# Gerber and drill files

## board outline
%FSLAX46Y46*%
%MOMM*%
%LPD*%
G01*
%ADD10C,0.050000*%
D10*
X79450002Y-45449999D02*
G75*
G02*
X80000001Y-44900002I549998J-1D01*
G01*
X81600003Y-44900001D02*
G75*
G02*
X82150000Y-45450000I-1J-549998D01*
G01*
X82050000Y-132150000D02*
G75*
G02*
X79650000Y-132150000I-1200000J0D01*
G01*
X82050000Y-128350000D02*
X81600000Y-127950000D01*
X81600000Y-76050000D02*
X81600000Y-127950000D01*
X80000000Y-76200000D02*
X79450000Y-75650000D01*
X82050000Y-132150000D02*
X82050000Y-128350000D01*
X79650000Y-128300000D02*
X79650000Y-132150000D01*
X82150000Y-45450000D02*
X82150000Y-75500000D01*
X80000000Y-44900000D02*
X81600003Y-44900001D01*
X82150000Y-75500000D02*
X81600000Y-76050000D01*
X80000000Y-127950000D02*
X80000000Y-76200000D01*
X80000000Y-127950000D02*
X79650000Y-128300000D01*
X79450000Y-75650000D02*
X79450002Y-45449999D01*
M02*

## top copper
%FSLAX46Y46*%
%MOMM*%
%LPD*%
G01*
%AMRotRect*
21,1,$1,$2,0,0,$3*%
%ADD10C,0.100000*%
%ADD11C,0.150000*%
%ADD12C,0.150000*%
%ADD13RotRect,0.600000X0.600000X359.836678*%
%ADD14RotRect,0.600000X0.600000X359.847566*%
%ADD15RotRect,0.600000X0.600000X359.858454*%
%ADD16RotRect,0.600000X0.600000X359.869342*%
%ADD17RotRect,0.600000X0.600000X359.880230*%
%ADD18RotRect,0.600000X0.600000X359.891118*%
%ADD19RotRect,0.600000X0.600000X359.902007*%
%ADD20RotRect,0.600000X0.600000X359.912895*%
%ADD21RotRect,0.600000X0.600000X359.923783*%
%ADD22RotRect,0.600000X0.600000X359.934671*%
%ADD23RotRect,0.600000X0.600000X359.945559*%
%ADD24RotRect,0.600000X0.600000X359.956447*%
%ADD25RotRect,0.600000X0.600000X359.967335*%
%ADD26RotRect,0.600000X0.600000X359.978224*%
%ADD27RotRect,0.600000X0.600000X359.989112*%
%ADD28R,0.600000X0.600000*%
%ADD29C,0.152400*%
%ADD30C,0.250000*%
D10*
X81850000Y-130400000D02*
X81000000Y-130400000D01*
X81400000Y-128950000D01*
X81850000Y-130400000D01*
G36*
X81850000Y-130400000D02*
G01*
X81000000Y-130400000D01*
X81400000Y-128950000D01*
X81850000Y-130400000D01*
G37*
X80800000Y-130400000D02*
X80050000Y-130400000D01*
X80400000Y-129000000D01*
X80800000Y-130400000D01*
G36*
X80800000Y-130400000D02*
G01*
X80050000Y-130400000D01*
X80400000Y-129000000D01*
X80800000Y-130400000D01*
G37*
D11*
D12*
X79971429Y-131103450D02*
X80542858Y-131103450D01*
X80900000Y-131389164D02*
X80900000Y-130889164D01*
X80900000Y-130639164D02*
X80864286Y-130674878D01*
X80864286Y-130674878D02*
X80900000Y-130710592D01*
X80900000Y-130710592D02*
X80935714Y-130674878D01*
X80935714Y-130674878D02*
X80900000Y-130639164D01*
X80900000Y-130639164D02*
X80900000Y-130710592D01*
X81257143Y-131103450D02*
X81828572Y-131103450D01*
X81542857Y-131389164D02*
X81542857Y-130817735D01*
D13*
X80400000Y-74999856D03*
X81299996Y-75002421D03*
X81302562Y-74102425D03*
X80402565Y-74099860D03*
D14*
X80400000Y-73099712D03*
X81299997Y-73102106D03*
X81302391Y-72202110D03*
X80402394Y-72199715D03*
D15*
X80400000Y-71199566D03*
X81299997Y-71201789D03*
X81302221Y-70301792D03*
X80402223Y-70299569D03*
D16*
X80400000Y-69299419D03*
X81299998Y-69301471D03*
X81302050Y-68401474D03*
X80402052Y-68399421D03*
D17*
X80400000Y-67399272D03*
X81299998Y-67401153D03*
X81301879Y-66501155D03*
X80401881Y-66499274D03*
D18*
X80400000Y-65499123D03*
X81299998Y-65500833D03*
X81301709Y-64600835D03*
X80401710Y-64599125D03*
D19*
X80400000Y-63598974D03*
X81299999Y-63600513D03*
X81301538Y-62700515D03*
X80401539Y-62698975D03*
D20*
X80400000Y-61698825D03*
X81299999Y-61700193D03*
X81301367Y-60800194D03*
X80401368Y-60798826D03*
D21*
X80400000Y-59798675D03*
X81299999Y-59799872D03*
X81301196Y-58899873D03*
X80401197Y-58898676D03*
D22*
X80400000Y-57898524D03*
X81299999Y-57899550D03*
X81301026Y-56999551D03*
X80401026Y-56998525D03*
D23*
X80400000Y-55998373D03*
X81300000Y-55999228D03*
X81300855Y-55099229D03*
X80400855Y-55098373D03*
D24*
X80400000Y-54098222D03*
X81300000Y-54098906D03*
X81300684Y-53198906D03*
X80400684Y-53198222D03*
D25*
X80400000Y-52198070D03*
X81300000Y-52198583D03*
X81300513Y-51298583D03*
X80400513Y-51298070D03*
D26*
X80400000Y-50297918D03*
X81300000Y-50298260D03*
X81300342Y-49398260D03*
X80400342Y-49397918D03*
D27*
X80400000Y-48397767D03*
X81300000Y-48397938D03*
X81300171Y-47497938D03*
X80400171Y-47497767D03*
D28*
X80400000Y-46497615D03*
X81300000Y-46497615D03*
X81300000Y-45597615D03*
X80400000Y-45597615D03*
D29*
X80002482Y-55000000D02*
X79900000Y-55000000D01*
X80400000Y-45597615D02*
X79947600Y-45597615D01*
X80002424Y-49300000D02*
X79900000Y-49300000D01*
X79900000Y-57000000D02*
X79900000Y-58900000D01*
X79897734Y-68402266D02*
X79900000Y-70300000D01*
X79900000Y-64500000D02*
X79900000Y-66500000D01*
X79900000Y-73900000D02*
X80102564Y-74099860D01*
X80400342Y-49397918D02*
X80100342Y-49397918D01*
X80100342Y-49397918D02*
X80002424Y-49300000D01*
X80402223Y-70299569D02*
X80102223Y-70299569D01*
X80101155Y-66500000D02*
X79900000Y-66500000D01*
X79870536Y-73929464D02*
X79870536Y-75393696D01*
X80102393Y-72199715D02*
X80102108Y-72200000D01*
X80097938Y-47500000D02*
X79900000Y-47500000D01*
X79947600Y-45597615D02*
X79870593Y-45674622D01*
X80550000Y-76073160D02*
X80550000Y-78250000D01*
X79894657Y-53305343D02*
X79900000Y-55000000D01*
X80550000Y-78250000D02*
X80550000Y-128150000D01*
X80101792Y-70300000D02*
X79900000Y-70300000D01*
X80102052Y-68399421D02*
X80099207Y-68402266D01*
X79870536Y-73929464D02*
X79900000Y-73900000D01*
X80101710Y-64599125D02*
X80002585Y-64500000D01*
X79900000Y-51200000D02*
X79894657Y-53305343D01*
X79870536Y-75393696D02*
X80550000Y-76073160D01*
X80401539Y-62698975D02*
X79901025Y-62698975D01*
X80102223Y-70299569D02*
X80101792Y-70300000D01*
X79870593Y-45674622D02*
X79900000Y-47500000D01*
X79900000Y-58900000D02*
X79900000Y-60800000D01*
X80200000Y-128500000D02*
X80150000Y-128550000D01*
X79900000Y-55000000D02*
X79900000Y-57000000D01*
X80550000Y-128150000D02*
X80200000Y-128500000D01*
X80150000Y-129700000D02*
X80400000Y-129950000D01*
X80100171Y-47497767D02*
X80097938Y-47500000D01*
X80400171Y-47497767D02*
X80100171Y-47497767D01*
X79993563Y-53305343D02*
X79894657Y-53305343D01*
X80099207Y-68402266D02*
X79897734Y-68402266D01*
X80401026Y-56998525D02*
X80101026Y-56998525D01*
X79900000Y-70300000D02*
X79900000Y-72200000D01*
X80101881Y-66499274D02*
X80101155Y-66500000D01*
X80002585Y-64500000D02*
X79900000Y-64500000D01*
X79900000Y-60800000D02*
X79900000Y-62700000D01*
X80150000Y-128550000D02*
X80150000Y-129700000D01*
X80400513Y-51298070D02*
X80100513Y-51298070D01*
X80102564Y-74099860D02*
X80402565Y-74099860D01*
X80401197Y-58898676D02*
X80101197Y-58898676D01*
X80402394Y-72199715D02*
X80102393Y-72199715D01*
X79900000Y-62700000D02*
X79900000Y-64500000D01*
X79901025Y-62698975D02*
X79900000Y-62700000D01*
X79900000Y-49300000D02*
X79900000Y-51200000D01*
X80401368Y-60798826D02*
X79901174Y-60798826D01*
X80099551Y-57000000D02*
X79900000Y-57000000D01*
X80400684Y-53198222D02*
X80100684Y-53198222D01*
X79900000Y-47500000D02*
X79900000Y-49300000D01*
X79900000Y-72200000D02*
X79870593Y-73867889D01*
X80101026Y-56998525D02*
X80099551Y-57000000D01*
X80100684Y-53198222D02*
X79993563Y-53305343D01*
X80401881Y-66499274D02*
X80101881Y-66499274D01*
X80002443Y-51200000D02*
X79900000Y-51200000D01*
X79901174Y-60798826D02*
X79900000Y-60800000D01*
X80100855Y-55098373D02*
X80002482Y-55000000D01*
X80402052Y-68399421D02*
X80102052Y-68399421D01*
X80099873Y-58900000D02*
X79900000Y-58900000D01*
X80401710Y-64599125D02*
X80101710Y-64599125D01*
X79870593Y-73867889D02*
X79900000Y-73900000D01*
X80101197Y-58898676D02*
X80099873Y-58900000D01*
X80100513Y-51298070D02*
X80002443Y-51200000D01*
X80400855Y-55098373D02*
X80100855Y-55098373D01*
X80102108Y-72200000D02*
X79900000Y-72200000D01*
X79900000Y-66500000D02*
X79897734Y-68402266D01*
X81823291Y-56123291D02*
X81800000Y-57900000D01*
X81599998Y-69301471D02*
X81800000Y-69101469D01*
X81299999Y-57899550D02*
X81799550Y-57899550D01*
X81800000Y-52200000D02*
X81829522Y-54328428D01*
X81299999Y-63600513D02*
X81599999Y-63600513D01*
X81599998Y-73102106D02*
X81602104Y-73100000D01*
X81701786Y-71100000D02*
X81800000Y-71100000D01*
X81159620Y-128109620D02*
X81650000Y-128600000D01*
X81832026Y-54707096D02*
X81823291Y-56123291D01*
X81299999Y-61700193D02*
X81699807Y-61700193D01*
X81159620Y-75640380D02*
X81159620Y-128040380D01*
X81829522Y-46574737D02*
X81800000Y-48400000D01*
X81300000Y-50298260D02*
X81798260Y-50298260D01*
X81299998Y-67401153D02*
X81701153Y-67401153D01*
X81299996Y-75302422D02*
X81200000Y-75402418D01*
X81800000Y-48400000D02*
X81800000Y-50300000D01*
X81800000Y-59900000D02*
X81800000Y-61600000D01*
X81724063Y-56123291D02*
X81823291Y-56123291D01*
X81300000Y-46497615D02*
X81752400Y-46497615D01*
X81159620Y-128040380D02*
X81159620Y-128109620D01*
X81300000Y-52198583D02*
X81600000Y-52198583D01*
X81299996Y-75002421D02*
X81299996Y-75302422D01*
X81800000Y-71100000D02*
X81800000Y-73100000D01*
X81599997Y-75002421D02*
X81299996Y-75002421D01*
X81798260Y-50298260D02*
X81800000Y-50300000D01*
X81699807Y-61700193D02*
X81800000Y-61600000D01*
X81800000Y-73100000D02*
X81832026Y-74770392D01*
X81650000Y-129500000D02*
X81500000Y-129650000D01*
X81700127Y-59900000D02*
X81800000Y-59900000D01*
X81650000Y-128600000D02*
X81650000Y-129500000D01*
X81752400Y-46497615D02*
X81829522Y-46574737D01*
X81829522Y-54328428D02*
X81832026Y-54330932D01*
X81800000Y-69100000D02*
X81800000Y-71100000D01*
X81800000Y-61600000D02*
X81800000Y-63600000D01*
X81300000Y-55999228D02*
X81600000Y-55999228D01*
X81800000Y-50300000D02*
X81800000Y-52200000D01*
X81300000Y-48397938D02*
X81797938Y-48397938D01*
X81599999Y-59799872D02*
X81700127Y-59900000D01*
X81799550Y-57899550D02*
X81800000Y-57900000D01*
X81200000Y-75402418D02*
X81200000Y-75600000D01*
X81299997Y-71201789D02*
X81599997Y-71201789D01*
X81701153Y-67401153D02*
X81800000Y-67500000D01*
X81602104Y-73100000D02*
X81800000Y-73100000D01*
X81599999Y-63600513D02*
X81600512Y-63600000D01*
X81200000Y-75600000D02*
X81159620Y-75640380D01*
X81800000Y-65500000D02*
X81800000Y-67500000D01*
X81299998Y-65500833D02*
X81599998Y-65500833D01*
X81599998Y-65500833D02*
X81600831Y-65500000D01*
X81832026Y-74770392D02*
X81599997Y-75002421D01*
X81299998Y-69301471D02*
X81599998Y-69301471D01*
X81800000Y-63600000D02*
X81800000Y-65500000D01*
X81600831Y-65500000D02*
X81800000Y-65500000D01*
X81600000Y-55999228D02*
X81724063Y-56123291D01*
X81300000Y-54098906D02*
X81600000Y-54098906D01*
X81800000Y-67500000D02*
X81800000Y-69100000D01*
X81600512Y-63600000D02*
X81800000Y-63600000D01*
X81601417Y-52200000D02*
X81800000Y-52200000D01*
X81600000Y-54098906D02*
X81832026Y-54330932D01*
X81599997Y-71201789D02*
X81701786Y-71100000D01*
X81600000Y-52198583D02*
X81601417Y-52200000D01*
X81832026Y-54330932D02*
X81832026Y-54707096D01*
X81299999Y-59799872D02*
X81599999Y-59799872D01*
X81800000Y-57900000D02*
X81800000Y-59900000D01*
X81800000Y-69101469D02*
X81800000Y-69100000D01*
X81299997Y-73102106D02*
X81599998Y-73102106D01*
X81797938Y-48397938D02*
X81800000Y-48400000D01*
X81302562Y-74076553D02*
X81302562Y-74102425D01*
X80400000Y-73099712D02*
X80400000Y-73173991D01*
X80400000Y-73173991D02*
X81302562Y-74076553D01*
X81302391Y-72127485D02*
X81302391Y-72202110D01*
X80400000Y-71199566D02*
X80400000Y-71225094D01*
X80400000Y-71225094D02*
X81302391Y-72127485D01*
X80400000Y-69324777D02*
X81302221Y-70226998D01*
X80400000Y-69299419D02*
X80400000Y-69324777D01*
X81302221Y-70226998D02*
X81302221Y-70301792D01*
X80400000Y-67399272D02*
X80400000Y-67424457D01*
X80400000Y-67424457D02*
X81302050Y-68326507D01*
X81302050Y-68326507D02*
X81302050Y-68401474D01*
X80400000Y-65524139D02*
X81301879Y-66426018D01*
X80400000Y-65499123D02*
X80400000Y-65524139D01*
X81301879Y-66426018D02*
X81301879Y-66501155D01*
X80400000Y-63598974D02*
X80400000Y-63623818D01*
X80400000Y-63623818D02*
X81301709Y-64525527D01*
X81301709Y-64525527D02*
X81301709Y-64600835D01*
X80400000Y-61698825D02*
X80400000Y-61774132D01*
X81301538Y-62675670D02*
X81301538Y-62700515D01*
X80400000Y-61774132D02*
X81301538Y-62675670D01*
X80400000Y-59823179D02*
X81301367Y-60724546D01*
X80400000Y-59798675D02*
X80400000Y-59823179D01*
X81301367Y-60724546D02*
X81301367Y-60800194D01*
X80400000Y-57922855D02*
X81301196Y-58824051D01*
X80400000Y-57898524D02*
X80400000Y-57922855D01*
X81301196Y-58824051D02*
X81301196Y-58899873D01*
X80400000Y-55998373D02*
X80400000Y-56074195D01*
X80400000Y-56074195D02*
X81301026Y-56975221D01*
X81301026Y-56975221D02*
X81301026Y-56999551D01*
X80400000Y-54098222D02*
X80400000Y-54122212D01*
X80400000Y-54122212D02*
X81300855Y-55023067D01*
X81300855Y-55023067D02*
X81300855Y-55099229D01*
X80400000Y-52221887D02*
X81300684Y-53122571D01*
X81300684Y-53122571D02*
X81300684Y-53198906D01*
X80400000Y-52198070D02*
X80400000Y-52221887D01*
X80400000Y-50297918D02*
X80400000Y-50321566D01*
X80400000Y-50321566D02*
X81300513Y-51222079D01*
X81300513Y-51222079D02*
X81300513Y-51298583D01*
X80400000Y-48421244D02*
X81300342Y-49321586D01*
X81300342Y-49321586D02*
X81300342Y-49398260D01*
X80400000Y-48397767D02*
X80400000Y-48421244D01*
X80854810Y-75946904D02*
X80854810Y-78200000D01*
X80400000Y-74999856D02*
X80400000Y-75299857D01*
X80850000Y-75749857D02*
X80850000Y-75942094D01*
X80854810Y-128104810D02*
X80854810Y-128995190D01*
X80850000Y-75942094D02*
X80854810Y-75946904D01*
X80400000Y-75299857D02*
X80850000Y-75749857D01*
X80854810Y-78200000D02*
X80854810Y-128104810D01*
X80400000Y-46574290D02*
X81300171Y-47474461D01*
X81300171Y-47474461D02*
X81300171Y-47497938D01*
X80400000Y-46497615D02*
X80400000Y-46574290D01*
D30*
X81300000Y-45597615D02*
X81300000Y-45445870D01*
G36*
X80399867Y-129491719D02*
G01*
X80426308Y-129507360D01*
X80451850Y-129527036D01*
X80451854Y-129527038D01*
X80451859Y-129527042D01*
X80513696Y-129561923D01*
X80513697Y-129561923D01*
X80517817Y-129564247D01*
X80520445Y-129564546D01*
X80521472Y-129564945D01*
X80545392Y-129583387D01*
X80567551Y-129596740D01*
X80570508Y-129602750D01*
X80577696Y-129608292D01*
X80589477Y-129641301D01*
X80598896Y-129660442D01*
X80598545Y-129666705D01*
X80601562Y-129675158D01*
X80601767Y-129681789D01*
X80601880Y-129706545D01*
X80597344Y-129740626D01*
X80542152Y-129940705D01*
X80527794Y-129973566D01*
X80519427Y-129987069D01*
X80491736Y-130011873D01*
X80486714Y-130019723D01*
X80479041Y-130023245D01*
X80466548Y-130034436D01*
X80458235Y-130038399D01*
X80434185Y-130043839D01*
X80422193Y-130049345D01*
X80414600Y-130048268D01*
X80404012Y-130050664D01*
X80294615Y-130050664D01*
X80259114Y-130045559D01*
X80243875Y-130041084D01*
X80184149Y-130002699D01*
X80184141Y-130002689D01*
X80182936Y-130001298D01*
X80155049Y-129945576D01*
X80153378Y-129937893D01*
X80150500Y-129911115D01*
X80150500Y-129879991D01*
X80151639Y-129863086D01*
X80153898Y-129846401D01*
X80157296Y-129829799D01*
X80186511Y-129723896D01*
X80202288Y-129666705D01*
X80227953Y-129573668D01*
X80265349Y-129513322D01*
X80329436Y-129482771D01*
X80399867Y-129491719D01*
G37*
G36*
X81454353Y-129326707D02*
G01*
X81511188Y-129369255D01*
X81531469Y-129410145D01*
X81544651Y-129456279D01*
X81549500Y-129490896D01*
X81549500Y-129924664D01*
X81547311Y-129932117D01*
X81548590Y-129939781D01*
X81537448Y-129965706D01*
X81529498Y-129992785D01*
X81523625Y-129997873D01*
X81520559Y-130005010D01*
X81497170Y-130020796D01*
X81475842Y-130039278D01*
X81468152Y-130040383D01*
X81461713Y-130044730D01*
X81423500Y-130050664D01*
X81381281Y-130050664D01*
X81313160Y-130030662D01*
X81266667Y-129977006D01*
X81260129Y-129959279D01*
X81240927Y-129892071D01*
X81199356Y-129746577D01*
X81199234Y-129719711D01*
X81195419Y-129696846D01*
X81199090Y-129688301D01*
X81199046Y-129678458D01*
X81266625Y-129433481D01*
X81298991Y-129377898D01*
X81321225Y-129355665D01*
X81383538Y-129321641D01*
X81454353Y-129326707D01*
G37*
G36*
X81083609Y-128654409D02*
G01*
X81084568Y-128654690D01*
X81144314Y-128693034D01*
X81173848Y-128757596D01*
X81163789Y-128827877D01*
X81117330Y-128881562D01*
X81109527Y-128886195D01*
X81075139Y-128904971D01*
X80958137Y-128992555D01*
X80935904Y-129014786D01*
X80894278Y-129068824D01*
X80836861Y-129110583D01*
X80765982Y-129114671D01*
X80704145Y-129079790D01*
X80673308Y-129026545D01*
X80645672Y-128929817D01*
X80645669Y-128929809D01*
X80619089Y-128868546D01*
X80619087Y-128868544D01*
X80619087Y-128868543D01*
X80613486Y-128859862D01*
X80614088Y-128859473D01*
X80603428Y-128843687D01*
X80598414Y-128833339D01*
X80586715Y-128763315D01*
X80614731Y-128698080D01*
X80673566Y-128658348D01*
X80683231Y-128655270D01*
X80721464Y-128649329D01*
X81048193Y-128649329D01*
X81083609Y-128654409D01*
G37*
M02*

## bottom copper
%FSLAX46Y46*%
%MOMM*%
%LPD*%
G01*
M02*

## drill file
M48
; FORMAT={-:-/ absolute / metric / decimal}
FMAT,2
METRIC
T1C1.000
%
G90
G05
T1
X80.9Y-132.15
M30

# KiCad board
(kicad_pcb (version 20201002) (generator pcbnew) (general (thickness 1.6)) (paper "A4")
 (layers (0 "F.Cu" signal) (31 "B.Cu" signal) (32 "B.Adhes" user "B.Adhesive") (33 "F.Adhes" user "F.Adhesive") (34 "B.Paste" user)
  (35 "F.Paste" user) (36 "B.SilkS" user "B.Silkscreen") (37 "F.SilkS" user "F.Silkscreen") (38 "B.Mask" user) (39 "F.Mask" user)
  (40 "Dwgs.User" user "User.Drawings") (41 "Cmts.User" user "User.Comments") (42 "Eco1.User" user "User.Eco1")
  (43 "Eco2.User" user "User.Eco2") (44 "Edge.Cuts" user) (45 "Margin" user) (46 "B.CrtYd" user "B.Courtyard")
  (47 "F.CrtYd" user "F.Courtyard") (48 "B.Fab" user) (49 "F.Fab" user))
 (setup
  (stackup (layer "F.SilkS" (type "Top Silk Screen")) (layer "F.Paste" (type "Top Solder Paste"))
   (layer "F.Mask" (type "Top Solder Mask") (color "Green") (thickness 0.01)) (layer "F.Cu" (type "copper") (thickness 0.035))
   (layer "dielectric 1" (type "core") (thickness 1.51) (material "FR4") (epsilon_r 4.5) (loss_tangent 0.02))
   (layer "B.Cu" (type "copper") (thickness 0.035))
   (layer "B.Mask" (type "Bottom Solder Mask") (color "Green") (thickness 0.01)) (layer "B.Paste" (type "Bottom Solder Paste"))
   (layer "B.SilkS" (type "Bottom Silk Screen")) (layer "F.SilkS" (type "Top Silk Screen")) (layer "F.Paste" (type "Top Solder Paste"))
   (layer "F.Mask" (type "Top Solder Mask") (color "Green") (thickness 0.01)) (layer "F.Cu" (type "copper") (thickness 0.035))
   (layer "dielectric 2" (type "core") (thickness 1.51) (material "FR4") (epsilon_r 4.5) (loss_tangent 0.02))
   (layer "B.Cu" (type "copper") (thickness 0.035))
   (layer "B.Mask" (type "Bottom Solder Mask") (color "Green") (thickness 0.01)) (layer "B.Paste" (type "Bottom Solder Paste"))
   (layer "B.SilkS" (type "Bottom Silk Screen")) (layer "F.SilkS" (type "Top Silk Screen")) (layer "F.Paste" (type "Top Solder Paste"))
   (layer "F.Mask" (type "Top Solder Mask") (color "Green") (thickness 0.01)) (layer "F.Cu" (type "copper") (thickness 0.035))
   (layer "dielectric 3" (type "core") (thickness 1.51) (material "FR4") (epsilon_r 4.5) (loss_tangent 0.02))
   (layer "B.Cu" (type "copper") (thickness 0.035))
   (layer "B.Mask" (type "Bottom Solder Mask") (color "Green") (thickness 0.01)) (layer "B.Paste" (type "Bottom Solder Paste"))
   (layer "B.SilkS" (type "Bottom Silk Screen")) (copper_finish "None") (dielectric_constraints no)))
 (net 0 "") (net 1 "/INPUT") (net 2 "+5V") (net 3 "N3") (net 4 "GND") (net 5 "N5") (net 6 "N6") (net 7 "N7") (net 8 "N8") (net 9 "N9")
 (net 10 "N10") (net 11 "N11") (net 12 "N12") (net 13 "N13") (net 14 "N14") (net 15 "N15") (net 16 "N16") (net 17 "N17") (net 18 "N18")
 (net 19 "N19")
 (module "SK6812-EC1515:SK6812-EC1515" (layer "F.Cu") (at 80.4 74.999856 -0.1633223699)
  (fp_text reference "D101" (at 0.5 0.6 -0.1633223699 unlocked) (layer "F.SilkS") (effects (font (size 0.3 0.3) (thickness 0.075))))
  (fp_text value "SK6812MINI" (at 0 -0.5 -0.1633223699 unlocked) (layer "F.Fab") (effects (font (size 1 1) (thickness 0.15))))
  (pad "1" smd rect (at 0 0 359.8366776) (size 0.6 0.6) (layers "F.Cu" "F.Paste" "F.Mask") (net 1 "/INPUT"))
  (pad "2" smd rect (at 0.9 0 359.8366776) (size 0.6 0.6) (layers "F.Cu" "F.Paste" "F.Mask") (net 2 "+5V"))
  (pad "3" smd rect (at 0.9 -0.9 359.8366776) (size 0.6 0.6) (layers "F.Cu" "F.Paste" "F.Mask") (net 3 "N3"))
  (pad "4" smd rect (at 0 -0.9 359.8366776) (size 0.6 0.6) (layers "F.Cu" "F.Paste" "F.Mask") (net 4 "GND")))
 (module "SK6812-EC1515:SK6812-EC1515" (layer "F.Cu") (at 80.4 73.099712 -0.1524342119)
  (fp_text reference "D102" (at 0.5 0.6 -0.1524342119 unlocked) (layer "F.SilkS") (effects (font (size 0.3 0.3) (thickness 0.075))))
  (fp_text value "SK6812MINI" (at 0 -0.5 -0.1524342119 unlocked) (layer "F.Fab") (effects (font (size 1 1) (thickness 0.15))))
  (pad "1" smd rect (at 0 0 359.8475658) (size 0.6 0.6) (layers "F.Cu" "F.Paste" "F.Mask") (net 3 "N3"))
  (pad "2" smd rect (at 0.9 0 359.8475658) (size 0.6 0.6) (layers "F.Cu" "F.Paste" "F.Mask") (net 2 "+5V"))
  (pad "3" smd rect (at 0.9 -0.9 359.8475658) (size 0.6 0.6) (layers "F.Cu" "F.Paste" "F.Mask") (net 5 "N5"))
  (pad "4" smd rect (at 0 -0.9 359.8475658) (size 0.6 0.6) (layers "F.Cu" "F.Paste" "F.Mask") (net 4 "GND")))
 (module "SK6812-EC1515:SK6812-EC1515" (layer "F.Cu") (at 80.4 71.199566 -0.1415460539)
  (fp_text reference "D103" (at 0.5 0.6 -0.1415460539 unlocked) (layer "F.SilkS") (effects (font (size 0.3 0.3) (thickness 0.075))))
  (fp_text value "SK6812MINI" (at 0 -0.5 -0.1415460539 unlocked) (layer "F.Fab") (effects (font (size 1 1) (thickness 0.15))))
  (pad "1" smd rect (at 0 0 359.8584539) (size 0.6 0.6) (layers "F.Cu" "F.Paste" "F.Mask") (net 5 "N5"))
  (pad "2" smd rect (at 0.9 0 359.8584539) (size 0.6 0.6) (layers "F.Cu" "F.Paste" "F.Mask") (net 2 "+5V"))
  (pad "3" smd rect (at 0.9 -0.9 359.8584539) (size 0.6 0.6) (layers "F.Cu" "F.Paste" "F.Mask") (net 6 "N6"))
  (pad "4" smd rect (at 0 -0.9 359.8584539) (size 0.6 0.6) (layers "F.Cu" "F.Paste" "F.Mask") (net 4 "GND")))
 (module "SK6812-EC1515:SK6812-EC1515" (layer "F.Cu") (at 80.4 69.299419 -0.1306578959)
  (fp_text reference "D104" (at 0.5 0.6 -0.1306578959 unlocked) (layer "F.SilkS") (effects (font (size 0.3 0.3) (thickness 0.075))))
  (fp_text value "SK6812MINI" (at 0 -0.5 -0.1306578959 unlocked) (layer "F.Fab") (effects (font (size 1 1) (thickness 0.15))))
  (pad "1" smd rect (at 0 0 359.8693421) (size 0.6 0.6) (layers "F.Cu" "F.Paste" "F.Mask") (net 6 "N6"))
  (pad "2" smd rect (at 0.9 0 359.8693421) (size 0.6 0.6) (layers "F.Cu" "F.Paste" "F.Mask") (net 2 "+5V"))
  (pad "3" smd rect (at 0.9 -0.9 359.8693421) (size 0.6 0.6) (layers "F.Cu" "F.Paste" "F.Mask") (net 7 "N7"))
  (pad "4" smd rect (at 0 -0.9 359.8693421) (size 0.6 0.6) (layers "F.Cu" "F.Paste" "F.Mask") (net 4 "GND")))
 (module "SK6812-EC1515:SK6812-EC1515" (layer "F.Cu") (at 80.4 67.399272 -0.1197697379)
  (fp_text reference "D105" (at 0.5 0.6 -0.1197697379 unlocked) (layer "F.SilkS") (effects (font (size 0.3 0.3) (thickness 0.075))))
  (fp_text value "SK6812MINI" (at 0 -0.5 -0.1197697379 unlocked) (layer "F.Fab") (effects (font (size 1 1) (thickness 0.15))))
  (pad "1" smd rect (at 0 0 359.8802303) (size 0.6 0.6) (layers "F.Cu" "F.Paste" "F.Mask") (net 7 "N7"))
  (pad "2" smd rect (at 0.9 0 359.8802303) (size 0.6 0.6) (layers "F.Cu" "F.Paste" "F.Mask") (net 2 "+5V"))
  (pad "3" smd rect (at 0.9 -0.9 359.8802303) (size 0.6 0.6) (layers "F.Cu" "F.Paste" "F.Mask") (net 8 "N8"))
  (pad "4" smd rect (at 0 -0.9 359.8802303) (size 0.6 0.6) (layers "F.Cu" "F.Paste" "F.Mask") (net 4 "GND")))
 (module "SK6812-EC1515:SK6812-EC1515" (layer "F.Cu") (at 80.4 65.499123 -0.1088815799)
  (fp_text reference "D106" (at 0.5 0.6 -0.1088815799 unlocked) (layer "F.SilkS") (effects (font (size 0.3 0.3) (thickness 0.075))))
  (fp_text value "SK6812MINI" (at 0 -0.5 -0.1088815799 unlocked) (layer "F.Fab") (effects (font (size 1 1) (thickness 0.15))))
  (pad "1" smd rect (at 0 0 359.8911184) (size 0.6 0.6) (layers "F.Cu" "F.Paste" "F.Mask") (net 8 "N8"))
  (pad "2" smd rect (at 0.9 0 359.8911184) (size 0.6 0.6) (layers "F.Cu" "F.Paste" "F.Mask") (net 2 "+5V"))
  (pad "3" smd rect (at 0.9 -0.9 359.8911184) (size 0.6 0.6) (layers "F.Cu" "F.Paste" "F.Mask") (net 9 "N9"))
  (pad "4" smd rect (at 0 -0.9 359.8911184) (size 0.6 0.6) (layers "F.Cu" "F.Paste" "F.Mask") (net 4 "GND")))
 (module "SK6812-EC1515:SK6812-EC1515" (layer "F.Cu") (at 80.4 63.598974 -0.09799342193)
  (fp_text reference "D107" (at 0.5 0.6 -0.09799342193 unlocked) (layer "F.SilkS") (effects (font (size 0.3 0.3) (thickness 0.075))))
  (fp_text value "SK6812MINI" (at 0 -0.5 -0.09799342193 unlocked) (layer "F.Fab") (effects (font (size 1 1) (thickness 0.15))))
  (pad "1" smd rect (at 0 0 359.9020066) (size 0.6 0.6) (layers "F.Cu" "F.Paste" "F.Mask") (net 9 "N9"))
  (pad "2" smd rect (at 0.9 0 359.9020066) (size 0.6 0.6) (layers "F.Cu" "F.Paste" "F.Mask") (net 2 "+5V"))
  (pad "3" smd rect (at 0.9 -0.9 359.9020066) (size 0.6 0.6) (layers "F.Cu" "F.Paste" "F.Mask") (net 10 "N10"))
  (pad "4" smd rect (at 0 -0.9 359.9020066) (size 0.6 0.6) (layers "F.Cu" "F.Paste" "F.Mask") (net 4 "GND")))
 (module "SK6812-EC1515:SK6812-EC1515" (layer "F.Cu") (at 80.4 61.698825 -0.08710526394)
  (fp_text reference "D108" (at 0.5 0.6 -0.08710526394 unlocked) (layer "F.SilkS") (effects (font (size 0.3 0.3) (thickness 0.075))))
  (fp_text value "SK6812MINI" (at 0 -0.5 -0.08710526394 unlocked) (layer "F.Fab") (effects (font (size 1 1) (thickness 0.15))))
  (pad "1" smd rect (at 0 0 359.9128947) (size 0.6 0.6) (layers "F.Cu" "F.Paste" "F.Mask") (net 10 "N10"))
  (pad "2" smd rect (at 0.9 0 359.9128947) (size 0.6 0.6) (layers "F.Cu" "F.Paste" "F.Mask") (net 2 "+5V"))
  (pad "3" smd rect (at 0.9 -0.9 359.9128947) (size 0.6 0.6) (layers "F.Cu" "F.Paste" "F.Mask") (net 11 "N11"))
  (pad "4" smd rect (at 0 -0.9 359.9128947) (size 0.6 0.6) (layers "F.Cu" "F.Paste" "F.Mask") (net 4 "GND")))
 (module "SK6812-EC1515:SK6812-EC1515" (layer "F.Cu") (at 80.4 59.798675 -0.07621710595)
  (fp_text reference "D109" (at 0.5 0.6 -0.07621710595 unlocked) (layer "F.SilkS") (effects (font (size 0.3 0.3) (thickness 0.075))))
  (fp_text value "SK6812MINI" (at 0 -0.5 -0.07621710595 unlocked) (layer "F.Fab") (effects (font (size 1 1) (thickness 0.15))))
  (pad "1" smd rect (at 0 0 359.9237829) (size 0.6 0.6) (layers "F.Cu" "F.Paste" "F.Mask") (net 11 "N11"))
  (pad "2" smd rect (at 0.9 0 359.9237829) (size 0.6 0.6) (layers "F.Cu" "F.Paste" "F.Mask") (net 2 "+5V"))
  (pad "3" smd rect (at 0.9 -0.9 359.9237829) (size 0.6 0.6) (layers "F.Cu" "F.Paste" "F.Mask") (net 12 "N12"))
  (pad "4" smd rect (at 0 -0.9 359.9237829) (size 0.6 0.6) (layers "F.Cu" "F.Paste" "F.Mask") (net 4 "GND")))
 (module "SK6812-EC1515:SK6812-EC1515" (layer "F.Cu") (at 80.4 57.898524 -0.06532894795)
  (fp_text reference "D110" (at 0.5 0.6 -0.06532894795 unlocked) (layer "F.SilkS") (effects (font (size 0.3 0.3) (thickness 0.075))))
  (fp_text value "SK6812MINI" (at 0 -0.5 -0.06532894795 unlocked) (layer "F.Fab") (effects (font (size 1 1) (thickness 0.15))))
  (pad "1" smd rect (at 0 0 359.9346711) (size 0.6 0.6) (layers "F.Cu" "F.Paste" "F.Mask") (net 12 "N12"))
  (pad "2" smd rect (at 0.9 0 359.9346711) (size 0.6 0.6) (layers "F.Cu" "F.Paste" "F.Mask") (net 2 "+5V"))
  (pad "3" smd rect (at 0.9 -0.9 359.9346711) (size 0.6 0.6) (layers "F.Cu" "F.Paste" "F.Mask") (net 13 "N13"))
  (pad "4" smd rect (at 0 -0.9 359.9346711) (size 0.6 0.6) (layers "F.Cu" "F.Paste" "F.Mask") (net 4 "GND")))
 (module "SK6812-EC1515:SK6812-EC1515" (layer "F.Cu") (at 80.4 55.998373 -0.05444078996)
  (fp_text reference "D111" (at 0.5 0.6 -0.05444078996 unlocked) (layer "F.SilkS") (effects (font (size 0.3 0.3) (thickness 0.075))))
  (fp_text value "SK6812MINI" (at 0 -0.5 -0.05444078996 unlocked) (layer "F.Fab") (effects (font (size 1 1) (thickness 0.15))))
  (pad "1" smd rect (at 0 0 359.9455592) (size 0.6 0.6) (layers "F.Cu" "F.Paste" "F.Mask") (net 13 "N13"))
  (pad "2" smd rect (at 0.9 0 359.9455592) (size 0.6 0.6) (layers "F.Cu" "F.Paste" "F.Mask") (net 2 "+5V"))
  (pad "3" smd rect (at 0.9 -0.9 359.9455592) (size 0.6 0.6) (layers "F.Cu" "F.Paste" "F.Mask") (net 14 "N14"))
  (pad "4" smd rect (at 0 -0.9 359.9455592) (size 0.6 0.6) (layers "F.Cu" "F.Paste" "F.Mask") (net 4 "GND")))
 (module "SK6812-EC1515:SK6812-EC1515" (layer "F.Cu") (at 80.4 54.098222 -0.04355263197)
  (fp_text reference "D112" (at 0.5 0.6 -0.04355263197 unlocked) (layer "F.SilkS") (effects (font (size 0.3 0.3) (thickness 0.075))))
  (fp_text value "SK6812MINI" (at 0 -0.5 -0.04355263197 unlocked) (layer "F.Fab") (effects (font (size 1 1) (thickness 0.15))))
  (pad "1" smd rect (at 0 0 359.9564474) (size 0.6 0.6) (layers "F.Cu" "F.Paste" "F.Mask") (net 14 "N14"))
  (pad "2" smd rect (at 0.9 0 359.9564474) (size 0.6 0.6) (layers "F.Cu" "F.Paste" "F.Mask") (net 2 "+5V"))
  (pad "3" smd rect (at 0.9 -0.9 359.9564474) (size 0.6 0.6) (layers "F.Cu" "F.Paste" "F.Mask") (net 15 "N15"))
  (pad "4" smd rect (at 0 -0.9 359.9564474) (size 0.6 0.6) (layers "F.Cu" "F.Paste" "F.Mask") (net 4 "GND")))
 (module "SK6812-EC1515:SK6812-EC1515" (layer "F.Cu") (at 80.4 52.19807 -0.03266447398)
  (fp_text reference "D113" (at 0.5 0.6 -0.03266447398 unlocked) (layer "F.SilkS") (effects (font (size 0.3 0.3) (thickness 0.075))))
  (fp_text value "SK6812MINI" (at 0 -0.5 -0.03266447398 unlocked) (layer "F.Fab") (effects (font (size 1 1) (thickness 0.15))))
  (pad "1" smd rect (at 0 0 359.9673355) (size 0.6 0.6) (layers "F.Cu" "F.Paste" "F.Mask") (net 15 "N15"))
  (pad "2" smd rect (at 0.9 0 359.9673355) (size 0.6 0.6) (layers "F.Cu" "F.Paste" "F.Mask") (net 2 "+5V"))
  (pad "3" smd rect (at 0.9 -0.9 359.9673355) (size 0.6 0.6) (layers "F.Cu" "F.Paste" "F.Mask") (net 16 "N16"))
  (pad "4" smd rect (at 0 -0.9 359.9673355) (size 0.6 0.6) (layers "F.Cu" "F.Paste" "F.Mask") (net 4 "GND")))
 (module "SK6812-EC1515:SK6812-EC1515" (layer "F.Cu") (at 80.4 50.297918 -0.02177631598)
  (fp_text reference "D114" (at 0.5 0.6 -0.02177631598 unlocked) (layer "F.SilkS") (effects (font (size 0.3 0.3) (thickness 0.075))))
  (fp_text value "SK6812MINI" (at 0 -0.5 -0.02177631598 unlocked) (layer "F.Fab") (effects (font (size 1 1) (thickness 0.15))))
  (pad "1" smd rect (at 0 0 359.9782237) (size 0.6 0.6) (layers "F.Cu" "F.Paste" "F.Mask") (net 16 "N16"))
  (pad "2" smd rect (at 0.9 0 359.9782237) (size 0.6 0.6) (layers "F.Cu" "F.Paste" "F.Mask") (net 2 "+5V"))
  (pad "3" smd rect (at 0.9 -0.9 359.9782237) (size 0.6 0.6) (layers "F.Cu" "F.Paste" "F.Mask") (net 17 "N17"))
  (pad "4" smd rect (at 0 -0.9 359.9782237) (size 0.6 0.6) (layers "F.Cu" "F.Paste" "F.Mask") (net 4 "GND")))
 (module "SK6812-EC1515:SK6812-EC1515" (layer "F.Cu") (at 80.4 48.397767 -0.01088815799)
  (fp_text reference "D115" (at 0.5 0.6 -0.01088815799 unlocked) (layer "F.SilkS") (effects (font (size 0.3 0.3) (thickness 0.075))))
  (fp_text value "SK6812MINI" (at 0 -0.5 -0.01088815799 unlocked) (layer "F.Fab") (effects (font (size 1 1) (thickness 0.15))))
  (pad "1" smd rect (at 0 0 359.9891118) (size 0.6 0.6) (layers "F.Cu" "F.Paste" "F.Mask") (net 17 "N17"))
  (pad "2" smd rect (at 0.9 0 359.9891118) (size 0.6 0.6) (layers "F.Cu" "F.Paste" "F.Mask") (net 2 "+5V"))
  (pad "3" smd rect (at 0.9 -0.9 359.9891118) (size 0.6 0.6) (layers "F.Cu" "F.Paste" "F.Mask") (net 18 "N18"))
  (pad "4" smd rect (at 0 -0.9 359.9891118) (size 0.6 0.6) (layers "F.Cu" "F.Paste" "F.Mask") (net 4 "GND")))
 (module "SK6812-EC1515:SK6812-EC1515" (layer "F.Cu") (at 80.4 46.497615)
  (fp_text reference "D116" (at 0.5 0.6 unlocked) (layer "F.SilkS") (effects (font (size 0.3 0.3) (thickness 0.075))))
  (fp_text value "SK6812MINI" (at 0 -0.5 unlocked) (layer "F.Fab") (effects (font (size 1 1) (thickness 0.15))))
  (pad "1" smd rect (at 0 0) (size 0.6 0.6) (layers "F.Cu" "F.Paste" "F.Mask") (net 18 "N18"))
  (pad "2" smd rect (at 0.9 0) (size 0.6 0.6) (layers "F.Cu" "F.Paste" "F.Mask") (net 2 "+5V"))
  (pad "3" smd rect (at 0.9 -0.9) (size 0.6 0.6) (layers "F.Cu" "F.Paste" "F.Mask"))
  (pad "4" smd rect (at 0 -0.9) (size 0.6 0.6) (layers "F.Cu" "F.Paste" "F.Mask") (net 4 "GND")))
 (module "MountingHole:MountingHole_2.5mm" (layer "F.Cu") (at 80.9 132.15)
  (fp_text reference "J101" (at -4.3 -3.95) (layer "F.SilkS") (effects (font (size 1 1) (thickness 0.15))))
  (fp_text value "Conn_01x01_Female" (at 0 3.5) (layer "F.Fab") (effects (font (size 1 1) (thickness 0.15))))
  (pad "" np_thru_hole circle (at 0 0) (size 1 1) (drill 1) (layers *.Cu *.Mask)))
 (gr_poly (pts (xy 81.85 130.4) (xy 81 130.4) (xy 81.4 128.95)) (layer "F.Cu") (width 0.1))
 (gr_poly (pts (xy 80.8 130.4) (xy 80.05 130.4) (xy 80.4 129)) (layer "F.Cu") (width 0.1))
 (gr_arc (start 80 45.45) (end 80.000001 44.900002) (angle -90) (layer "Edge.Cuts") (width 0.05))
 (gr_arc (start 81.600002 45.449999) (end 82.15 45.45) (angle -90) (layer "Edge.Cuts") (width 0.05))
 (gr_arc (start 80.85 132.15) (end 79.65 132.15) (angle -180) (layer "Edge.Cuts") (width 0.05))
 (gr_line (start 82.05 128.35) (end 81.6 127.95) (layer "Edge.Cuts") (width 0.05))
 (gr_line (start 81.6 76.05) (end 81.6 127.95) (layer "Edge.Cuts") (width 0.05))
 (gr_line (start 80 76.2) (end 79.45 75.65) (layer "Edge.Cuts") (width 0.05))
 (gr_line (start 82.05 132.15) (end 82.05 128.35) (layer "Edge.Cuts") (width 0.05))
 (gr_line (start 79.65 128.3) (end 79.65 132.15) (layer "Edge.Cuts") (width 0.05))
 (gr_line (start 82.15 45.45) (end 82.15 75.5) (layer "Edge.Cuts") (width 0.05))
 (gr_line (start 80 44.9) (end 81.600003 44.900001) (layer "Edge.Cuts") (width 0.05))
 (gr_line (start 82.15 75.5) (end 81.6 76.05) (layer "Edge.Cuts") (width 0.05))
 (gr_line (start 80 127.95) (end 80 76.2) (layer "Edge.Cuts") (width 0.05))
 (gr_line (start 80 127.95) (end 79.65 128.3) (layer "Edge.Cuts") (width 0.05))
 (gr_line (start 79.45 75.65) (end 79.450002 45.449999) (layer "Edge.Cuts") (width 0.05))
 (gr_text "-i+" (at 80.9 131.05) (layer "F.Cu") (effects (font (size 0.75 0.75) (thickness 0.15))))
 (segment (start 80.002482 55) (end 79.9 55) (width 0.1524) (layer "F.Cu") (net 4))
 (segment (start 80.4 45.597615) (end 79.9476 45.597615) (width 0.1524) (layer "F.Cu") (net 4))
 (segment (start 80.002424 49.3) (end 79.9 49.3) (width 0.1524) (layer "F.Cu") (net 4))
 (segment (start 79.9 57) (end 79.9 58.9) (width 0.1524) (layer "F.Cu") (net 4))
 (segment (start 79.897734 68.402266) (end 79.9 70.3) (width 0.1524) (layer "F.Cu") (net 4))
 (segment (start 79.9 64.5) (end 79.9 66.5) (width 0.1524) (layer "F.Cu") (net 4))
 (segment (start 79.9 73.9) (end 80.102564 74.09986) (width 0.1524) (layer "F.Cu") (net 4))
 (segment (start 80.400342 49.397918) (end 80.100342 49.397918) (width 0.1524) (layer "F.Cu") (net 4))
 (segment (start 80.100342 49.397918) (end 80.002424 49.3) (width 0.1524) (layer "F.Cu") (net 4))
 (segment (start 80.402223 70.299569) (end 80.102223 70.299569) (width 0.1524) (layer "F.Cu") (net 4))
 (segment (start 80.101155 66.5) (end 79.9 66.5) (width 0.1524) (layer "F.Cu") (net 4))
 (segment (start 79.870536 73.929464) (end 79.870536 75.393696) (width 0.1524) (layer "F.Cu") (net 4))
 (segment (start 80.102393 72.199715) (end 80.102108 72.2) (width 0.1524) (layer "F.Cu") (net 4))
 (segment (start 80.097938 47.5) (end 79.9 47.5) (width 0.1524) (layer "F.Cu") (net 4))
 (segment (start 79.9476 45.597615) (end 79.870593 45.674622) (width 0.1524) (layer "F.Cu") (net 4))
 (segment (start 80.55 76.07316) (end 80.55 78.25) (width 0.1524) (layer "F.Cu") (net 4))
 (segment (start 79.894657 53.305343) (end 79.9 55) (width 0.1524) (layer "F.Cu") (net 4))
 (segment (start 80.55 78.25) (end 80.55 128.15) (width 0.1524) (layer "F.Cu") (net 4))
 (segment (start 80.101792 70.3) (end 79.9 70.3) (width 0.1524) (layer "F.Cu") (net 4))
 (segment (start 80.102052 68.399421) (end 80.099207 68.402266) (width 0.1524) (layer "F.Cu") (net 4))
 (segment (start 79.870536 73.929464) (end 79.9 73.9) (width 0.1524) (layer "F.Cu") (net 4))
 (segment (start 80.10171 64.599125) (end 80.002585 64.5) (width 0.1524) (layer "F.Cu") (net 4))
 (segment (start 79.9 51.2) (end 79.894657 53.305343) (width 0.1524) (layer "F.Cu") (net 4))
 (segment (start 79.870536 75.393696) (end 80.55 76.07316) (width 0.1524) (layer "F.Cu") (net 4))
 (segment (start 80.401539 62.698975) (end 79.901025 62.698975) (width 0.1524) (layer "F.Cu") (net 4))
 (segment (start 80.102223 70.299569) (end 80.101792 70.3) (width 0.1524) (layer "F.Cu") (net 4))
 (segment (start 79.870593 45.674622) (end 79.9 47.5) (width 0.1524) (layer "F.Cu") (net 4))
 (segment (start 79.9 58.9) (end 79.9 60.8) (width 0.1524) (layer "F.Cu") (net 4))
 (segment (start 80.2 128.5) (end 80.15 128.55) (width 0.1524) (layer "F.Cu") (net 4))
 (segment (start 79.9 55) (end 79.9 57) (width 0.1524) (layer "F.Cu") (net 4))
 (segment (start 80.55 128.15) (end 80.2 128.5) (width 0.1524) (layer "F.Cu") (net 4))
 (segment (start 80.15 129.7) (end 80.4 129.95) (width 0.1524) (layer "F.Cu") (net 4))
 (segment (start 80.100171 47.497767) (end 80.097938 47.5) (width 0.1524) (layer "F.Cu") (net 4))
 (segment (start 80.400171 47.497767) (end 80.100171 47.497767) (width 0.1524) (layer "F.Cu") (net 4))
 (segment (start 79.993563 53.305343) (end 79.894657 53.305343) (width 0.1524) (layer "F.Cu") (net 4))
 (segment (start 80.099207 68.402266) (end 79.897734 68.402266) (width 0.1524) (layer "F.Cu") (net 4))
 (segment (start 80.401026 56.998525) (end 80.101026 56.998525) (width 0.1524) (layer "F.Cu") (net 4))
 (segment (start 79.9 70.3) (end 79.9 72.2) (width 0.1524) (layer "F.Cu") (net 4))
 (segment (start 80.101881 66.499274) (end 80.101155 66.5) (width 0.1524) (layer "F.Cu") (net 4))
 (segment (start 80.002585 64.5) (end 79.9 64.5) (width 0.1524) (layer "F.Cu") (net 4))
 (segment (start 79.9 60.8) (end 79.9 62.7) (width 0.1524) (layer "F.Cu") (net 4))
 (segment (start 80.15 128.55) (end 80.15 129.7) (width 0.1524) (layer "F.Cu") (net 4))
 (segment (start 80.400513 51.29807) (end 80.100513 51.29807) (width 0.1524) (layer "F.Cu") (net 4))
 (segment (start 80.102564 74.09986) (end 80.402565 74.09986) (width 0.1524) (layer "F.Cu") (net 4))
 (segment (start 80.401197 58.898676) (end 80.101197 58.898676) (width 0.1524) (layer "F.Cu") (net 4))
 (segment (start 80.402394 72.199715) (end 80.102393 72.199715) (width 0.1524) (layer "F.Cu") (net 4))
 (segment (start 79.9 62.7) (end 79.9 64.5) (width 0.1524) (layer "F.Cu") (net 4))
 (segment (start 79.901025 62.698975) (end 79.9 62.7) (width 0.1524) (layer "F.Cu") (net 4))
 (segment (start 79.9 49.3) (end 79.9 51.2) (width 0.1524) (layer "F.Cu") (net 4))
 (segment (start 80.401368 60.798826) (end 79.901174 60.798826) (width 0.1524) (layer "F.Cu") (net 4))
 (segment (start 80.099551 57) (end 79.9 57) (width 0.1524) (layer "F.Cu") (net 4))
 (segment (start 80.400684 53.198222) (end 80.100684 53.198222) (width 0.1524) (layer "F.Cu") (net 4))
 (segment (start 79.9 47.5) (end 79.9 49.3) (width 0.1524) (layer "F.Cu") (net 4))
 (segment (start 79.9 72.2) (end 79.870593 73.867889) (width 0.1524) (layer "F.Cu") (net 4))
 (segment (start 80.101026 56.998525) (end 80.099551 57) (width 0.1524) (layer "F.Cu") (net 4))
 (segment (start 80.100684 53.198222) (end 79.993563 53.305343) (width 0.1524) (layer "F.Cu") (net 4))
 (segment (start 80.401881 66.499274) (end 80.101881 66.499274) (width 0.1524) (layer "F.Cu") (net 4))
 (segment (start 80.002443 51.2) (end 79.9 51.2) (width 0.1524) (layer "F.Cu") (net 4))
 (segment (start 79.901174 60.798826) (end 79.9 60.8) (width 0.1524) (layer "F.Cu") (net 4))
 (segment (start 80.100855 55.098373) (end 80.002482 55) (width 0.1524) (layer "F.Cu") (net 4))
 (segment (start 80.402052 68.399421) (end 80.102052 68.399421) (width 0.1524) (layer "F.Cu") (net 4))
 (segment (start 80.099873 58.9) (end 79.9 58.9) (width 0.1524) (layer "F.Cu") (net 4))
 (segment (start 80.40171 64.599125) (end 80.10171 64.599125) (width 0.1524) (layer "F.Cu") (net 4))
 (segment (start 79.870593 73.867889) (end 79.9 73.9) (width 0.1524) (layer "F.Cu") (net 4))
 (segment (start 80.101197 58.898676) (end 80.099873 58.9) (width 0.1524) (layer "F.Cu") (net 4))
 (segment (start 80.100513 51.29807) (end 80.002443 51.2) (width 0.1524) (layer "F.Cu") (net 4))
 (segment (start 80.400855 55.098373) (end 80.100855 55.098373) (width 0.1524) (layer "F.Cu") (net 4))
 (segment (start 80.102108 72.2) (end 79.9 72.2) (width 0.1524) (layer "F.Cu") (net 4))
 (segment (start 79.9 66.5) (end 79.897734 68.402266) (width 0.1524) (layer "F.Cu") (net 4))
 (segment (start 81.823291 56.123291) (end 81.8 57.9) (width 0.1524) (layer "F.Cu") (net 2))
 (segment (start 81.599998 69.301471) (end 81.8 69.101469) (width 0.1524) (layer "F.Cu") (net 2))
 (segment (start 81.299999 57.89955) (end 81.79955 57.89955) (width 0.1524) (layer "F.Cu") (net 2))
 (segment (start 81.8 52.2) (end 81.829522 54.328428) (width 0.1524) (layer "F.Cu") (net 2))
 (segment (start 81.299999 63.600513) (end 81.599999 63.600513) (width 0.1524) (layer "F.Cu") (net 2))
 (segment (start 81.599998 73.102106) (end 81.602104 73.1) (width 0.1524) (layer "F.Cu") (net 2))
 (segment (start 81.701786 71.1) (end 81.8 71.1) (width 0.1524) (layer "F.Cu") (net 2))
 (segment (start 81.15962 128.10962) (end 81.65 128.6) (width 0.1524) (layer "F.Cu") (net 2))
 (segment (start 81.832026 54.707096) (end 81.823291 56.123291) (width 0.1524) (layer "F.Cu") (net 2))
 (segment (start 81.299999 61.700193) (end 81.699807 61.700193) (width 0.1524) (layer "F.Cu") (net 2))
 (segment (start 81.15962 75.64038) (end 81.15962 128.04038) (width 0.1524) (layer "F.Cu") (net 2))
 (segment (start 81.829522 46.574737) (end 81.8 48.4) (width 0.1524) (layer "F.Cu") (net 2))
 (segment (start 81.3 50.29826) (end 81.79826 50.29826) (width 0.1524) (layer "F.Cu") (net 2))
 (segment (start 81.299998 67.401153) (end 81.701153 67.401153) (width 0.1524) (layer "F.Cu") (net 2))
 (segment (start 81.299996 75.302422) (end 81.2 75.402418) (width 0.1524) (layer "F.Cu") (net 2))
 (segment (start 81.8 48.4) (end 81.8 50.3) (width 0.1524) (layer "F.Cu") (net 2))
 (segment (start 81.8 59.9) (end 81.8 61.6) (width 0.1524) (layer "F.Cu") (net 2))
 (segment (start 81.724063 56.123291) (end 81.823291 56.123291) (width 0.1524) (layer "F.Cu") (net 2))
 (segment (start 81.3 46.497615) (end 81.7524 46.497615) (width 0.1524) (layer "F.Cu") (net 2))
 (segment (start 81.15962 128.04038) (end 81.15962 128.10962) (width 0.1524) (layer "F.Cu") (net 2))
 (segment (start 81.3 52.198583) (end 81.6 52.198583) (width 0.1524) (layer "F.Cu") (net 2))
 (segment (start 81.299996 75.002421) (end 81.299996 75.302422) (width 0.1524) (layer "F.Cu") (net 2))
 (segment (start 81.8 71.1) (end 81.8 73.1) (width 0.1524) (layer "F.Cu") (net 2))
 (segment (start 81.599997 75.002421) (end 81.299996 75.002421) (width 0.1524) (layer "F.Cu") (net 2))
 (segment (start 81.79826 50.29826) (end 81.8 50.3) (width 0.1524) (layer "F.Cu") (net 2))
 (segment (start 81.699807 61.700193) (end 81.8 61.6) (width 0.1524) (layer "F.Cu") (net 2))
 (segment (start 81.8 73.1) (end 81.832026 74.770392) (width 0.1524) (layer "F.Cu") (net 2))
 (segment (start 81.65 129.5) (end 81.5 129.65) (width 0.1524) (layer "F.Cu") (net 2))
 (segment (start 81.700127 59.9) (end 81.8 59.9) (width 0.1524) (layer "F.Cu") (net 2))
 (segment (start 81.65 128.6) (end 81.65 129.5) (width 0.1524) (layer "F.Cu") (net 2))
 (segment (start 81.7524 46.497615) (end 81.829522 46.574737) (width 0.1524) (layer "F.Cu") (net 2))
 (segment (start 81.829522 54.328428) (end 81.832026 54.330932) (width 0.1524) (layer "F.Cu") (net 2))
 (segment (start 81.8 69.1) (end 81.8 71.1) (width 0.1524) (layer "F.Cu") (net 2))
 (segment (start 81.8 61.6) (end 81.8 63.6) (width 0.1524) (layer "F.Cu") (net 2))
 (segment (start 81.3 55.999228) (end 81.6 55.999228) (width 0.1524) (layer "F.Cu") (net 2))
 (segment (start 81.8 50.3) (end 81.8 52.2) (width 0.1524) (layer "F.Cu") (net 2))
 (segment (start 81.3 48.397938) (end 81.797938 48.397938) (width 0.1524) (layer "F.Cu") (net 2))
 (segment (start 81.599999 59.799872) (end 81.700127 59.9) (width 0.1524) (layer "F.Cu") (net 2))
 (segment (start 81.79955 57.89955) (end 81.8 57.9) (width 0.1524) (layer "F.Cu") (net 2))
 (segment (start 81.2 75.402418) (end 81.2 75.6) (width 0.1524) (layer "F.Cu") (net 2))
 (segment (start 81.299997 71.201789) (end 81.599997 71.201789) (width 0.1524) (layer "F.Cu") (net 2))
 (segment (start 81.701153 67.401153) (end 81.8 67.5) (width 0.1524) (layer "F.Cu") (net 2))
 (segment (start 81.602104 73.1) (end 81.8 73.1) (width 0.1524) (layer "F.Cu") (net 2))
 (segment (start 81.599999 63.600513) (end 81.600512 63.6) (width 0.1524) (layer "F.Cu") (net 2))
 (segment (start 81.2 75.6) (end 81.15962 75.64038) (width 0.1524) (layer "F.Cu") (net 2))
 (segment (start 81.8 65.5) (end 81.8 67.5) (width 0.1524) (layer "F.Cu") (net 2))
 (segment (start 81.299998 65.500833) (end 81.599998 65.500833) (width 0.1524) (layer "F.Cu") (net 2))
 (segment (start 81.599998 65.500833) (end 81.600831 65.5) (width 0.1524) (layer "F.Cu") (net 2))
 (segment (start 81.832026 74.770392) (end 81.599997 75.002421) (width 0.1524) (layer "F.Cu") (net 2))
 (segment (start 81.299998 69.301471) (end 81.599998 69.301471) (width 0.1524) (layer "F.Cu") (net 2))
 (segment (start 81.8 63.6) (end 81.8 65.5) (width 0.1524) (layer "F.Cu") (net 2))
 (segment (start 81.600831 65.5) (end 81.8 65.5) (width 0.1524) (layer "F.Cu") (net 2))
 (segment (start 81.6 55.999228) (end 81.724063 56.123291) (width 0.1524) (layer "F.Cu") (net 2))
 (segment (start 81.3 54.098906) (end 81.6 54.098906) (width 0.1524) (layer "F.Cu") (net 2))
 (segment (start 81.8 67.5) (end 81.8 69.1) (width 0.1524) (layer "F.Cu") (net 2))
 (segment (start 81.600512 63.6) (end 81.8 63.6) (width 0.1524) (layer "F.Cu") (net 2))
 (segment (start 81.601417 52.2) (end 81.8 52.2) (width 0.1524) (layer "F.Cu") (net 2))
 (segment (start 81.6 54.098906) (end 81.832026 54.330932) (width 0.1524) (layer "F.Cu") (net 2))
 (segment (start 81.599997 71.201789) (end 81.701786 71.1) (width 0.1524) (layer "F.Cu") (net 2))
 (segment (start 81.6 52.198583) (end 81.601417 52.2) (width 0.1524) (layer "F.Cu") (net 2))
 (segment (start 81.832026 54.330932) (end 81.832026 54.707096) (width 0.1524) (layer "F.Cu") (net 2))
 (segment (start 81.299999 59.799872) (end 81.599999 59.799872) (width 0.1524) (layer "F.Cu") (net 2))
 (segment (start 81.8 57.9) (end 81.8 59.9) (width 0.1524) (layer "F.Cu") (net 2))
 (segment (start 81.8 69.101469) (end 81.8 69.1) (width 0.1524) (layer "F.Cu") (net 2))
 (segment (start 81.299997 73.102106) (end 81.599998 73.102106) (width 0.1524) (layer "F.Cu") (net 2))
 (segment (start 81.797938 48.397938) (end 81.8 48.4) (width 0.1524) (layer "F.Cu") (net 2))
 (segment (start 81.302562 74.076553) (end 81.302562 74.102425) (width 0.1524) (layer "F.Cu") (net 3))
 (segment (start 80.4 73.099712) (end 80.4 73.173991) (width 0.1524) (layer "F.Cu") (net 3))
 (segment (start 80.4 73.173991) (end 81.302562 74.076553) (width 0.1524) (layer "F.Cu") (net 3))
 (segment (start 81.302391 72.127485) (end 81.302391 72.20211) (width 0.1524) (layer "F.Cu") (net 5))
 (segment (start 80.4 71.199566) (end 80.4 71.225094) (width 0.1524) (layer "F.Cu") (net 5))
 (segment (start 80.4 71.225094) (end 81.302391 72.127485) (width 0.1524) (layer "F.Cu") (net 5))
 (segment (start 80.4 69.324777) (end 81.302221 70.226998) (width 0.1524) (layer "F.Cu") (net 6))
 (segment (start 80.4 69.299419) (end 80.4 69.324777) (width 0.1524) (layer "F.Cu") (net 6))
 (segment (start 81.302221 70.226998) (end 81.302221 70.301792) (width 0.1524) (layer "F.Cu") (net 6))
 (segment (start 80.4 67.399272) (end 80.4 67.424457) (width 0.1524) (layer "F.Cu") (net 7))
 (segment (start 80.4 67.424457) (end 81.30205 68.326507) (width 0.1524) (layer "F.Cu") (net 7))
 (segment (start 81.30205 68.326507) (end 81.30205 68.401474) (width 0.1524) (layer "F.Cu") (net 7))
 (segment (start 80.4 65.524139) (end 81.301879 66.426018) (width 0.1524) (layer "F.Cu") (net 8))
 (segment (start 80.4 65.499123) (end 80.4 65.524139) (width 0.1524) (layer "F.Cu") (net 8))
 (segment (start 81.301879 66.426018) (end 81.301879 66.501155) (width 0.1524) (layer "F.Cu") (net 8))
 (segment (start 80.4 63.598974) (end 80.4 63.623818) (width 0.1524) (layer "F.Cu") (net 9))
 (segment (start 80.4 63.623818) (end 81.301709 64.525527) (width 0.1524) (layer "F.Cu") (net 9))
 (segment (start 81.301709 64.525527) (end 81.301709 64.600835) (width 0.1524) (layer "F.Cu") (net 9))
 (segment (start 80.4 61.698825) (end 80.4 61.774132) (width 0.1524) (layer "F.Cu") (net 10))
 (segment (start 81.301538 62.67567) (end 81.301538 62.700515) (width 0.1524) (layer "F.Cu") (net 10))
 (segment (start 80.4 61.774132) (end 81.301538 62.67567) (width 0.1524) (layer "F.Cu") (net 10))
 (segment (start 80.4 59.823179) (end 81.301367 60.724546) (width 0.1524) (layer "F.Cu") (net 11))
 (segment (start 80.4 59.798675) (end 80.4 59.823179) (width 0.1524) (layer "F.Cu") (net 11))
 (segment (start 81.301367 60.724546) (end 81.301367 60.800194) (width 0.1524) (layer "F.Cu") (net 11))
 (segment (start 80.4 57.922855) (end 81.301196 58.824051) (width 0.1524) (layer "F.Cu") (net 12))
 (segment (start 80.4 57.898524) (end 80.4 57.922855) (width 0.1524) (layer "F.Cu") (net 12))
 (segment (start 81.301196 58.824051) (end 81.301196 58.899873) (width 0.1524) (layer "F.Cu") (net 12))
 (segment (start 80.4 55.998373) (end 80.4 56.074195) (width 0.1524) (layer "F.Cu") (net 13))
 (segment (start 80.4 56.074195) (end 81.301026 56.975221) (width 0.1524) (layer "F.Cu") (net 13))
 (segment (start 81.301026 56.975221) (end 81.301026 56.999551) (width 0.1524) (layer "F.Cu") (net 13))
 (segment (start 80.4 54.098222) (end 80.4 54.122212) (width 0.1524) (layer "F.Cu") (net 14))
 (segment (start 80.4 54.122212) (end 81.300855 55.023067) (width 0.1524) (layer "F.Cu") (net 14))
 (segment (start 81.300855 55.023067) (end 81.300855 55.099229) (width 0.1524) (layer "F.Cu") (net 14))
 (segment (start 80.4 52.221887) (end 81.300684 53.122571) (width 0.1524) (layer "F.Cu") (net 15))
 (segment (start 81.300684 53.122571) (end 81.300684 53.198906) (width 0.1524) (layer "F.Cu") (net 15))
 (segment (start 80.4 52.19807) (end 80.4 52.221887) (width 0.1524) (layer "F.Cu") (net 15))
 (segment (start 80.4 50.297918) (end 80.4 50.321566) (width 0.1524) (layer "F.Cu") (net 16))
 (segment (start 80.4 50.321566) (end 81.300513 51.222079) (width 0.1524) (layer "F.Cu") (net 16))
 (segment (start 81.300513 51.222079) (end 81.300513 51.298583) (width 0.1524) (layer "F.Cu") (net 16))
 (segment (start 80.4 48.421244) (end 81.300342 49.321586) (width 0.1524) (layer "F.Cu") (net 17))
 (segment (start 81.300342 49.321586) (end 81.300342 49.39826) (width 0.1524) (layer "F.Cu") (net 17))
 (segment (start 80.4 48.397767) (end 80.4 48.421244) (width 0.1524) (layer "F.Cu") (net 17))
 (segment (start 80.85481 75.946904) (end 80.85481 78.2) (width 0.1524) (layer "F.Cu") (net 1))
 (segment (start 80.4 74.999856) (end 80.4 75.299857) (width 0.1524) (layer "F.Cu") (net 1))
 (segment (start 80.85 75.749857) (end 80.85 75.942094) (width 0.1524) (layer "F.Cu") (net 1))
 (segment (start 80.85481 128.10481) (end 80.85481 128.99519) (width 0.1524) (layer "F.Cu") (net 1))
 (segment (start 80.85 75.942094) (end 80.85481 75.946904) (width 0.1524) (layer "F.Cu") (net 1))
 (segment (start 80.4 75.299857) (end 80.85 75.749857) (width 0.1524) (layer "F.Cu") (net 1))
 (segment (start 80.85481 78.2) (end 80.85481 128.10481) (width 0.1524) (layer "F.Cu") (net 1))
 (segment (start 80.4 46.57429) (end 81.300171 47.474461) (width 0.1524) (layer "F.Cu") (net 18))
 (segment (start 81.300171 47.474461) (end 81.300171 47.497938) (width 0.1524) (layer "F.Cu") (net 18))
 (segment (start 80.4 46.497615) (end 80.4 46.57429) (width 0.1524) (layer "F.Cu") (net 18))
 (segment (start 81.3 45.597615) (end 81.3 45.44587) (width 0.25) (layer "F.Cu") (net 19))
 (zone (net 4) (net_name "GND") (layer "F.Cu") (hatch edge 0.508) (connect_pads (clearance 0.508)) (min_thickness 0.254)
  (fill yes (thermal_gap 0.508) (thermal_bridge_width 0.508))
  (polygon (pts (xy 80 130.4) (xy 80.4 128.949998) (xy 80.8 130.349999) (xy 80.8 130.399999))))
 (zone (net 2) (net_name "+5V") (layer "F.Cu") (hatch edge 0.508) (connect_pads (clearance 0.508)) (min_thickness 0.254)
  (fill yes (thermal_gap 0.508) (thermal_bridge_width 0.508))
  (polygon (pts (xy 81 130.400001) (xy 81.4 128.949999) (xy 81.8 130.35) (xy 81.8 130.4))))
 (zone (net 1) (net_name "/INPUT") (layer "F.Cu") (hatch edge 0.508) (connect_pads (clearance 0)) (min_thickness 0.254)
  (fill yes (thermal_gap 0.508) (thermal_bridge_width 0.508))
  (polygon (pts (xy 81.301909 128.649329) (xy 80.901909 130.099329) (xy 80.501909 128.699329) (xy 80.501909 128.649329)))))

